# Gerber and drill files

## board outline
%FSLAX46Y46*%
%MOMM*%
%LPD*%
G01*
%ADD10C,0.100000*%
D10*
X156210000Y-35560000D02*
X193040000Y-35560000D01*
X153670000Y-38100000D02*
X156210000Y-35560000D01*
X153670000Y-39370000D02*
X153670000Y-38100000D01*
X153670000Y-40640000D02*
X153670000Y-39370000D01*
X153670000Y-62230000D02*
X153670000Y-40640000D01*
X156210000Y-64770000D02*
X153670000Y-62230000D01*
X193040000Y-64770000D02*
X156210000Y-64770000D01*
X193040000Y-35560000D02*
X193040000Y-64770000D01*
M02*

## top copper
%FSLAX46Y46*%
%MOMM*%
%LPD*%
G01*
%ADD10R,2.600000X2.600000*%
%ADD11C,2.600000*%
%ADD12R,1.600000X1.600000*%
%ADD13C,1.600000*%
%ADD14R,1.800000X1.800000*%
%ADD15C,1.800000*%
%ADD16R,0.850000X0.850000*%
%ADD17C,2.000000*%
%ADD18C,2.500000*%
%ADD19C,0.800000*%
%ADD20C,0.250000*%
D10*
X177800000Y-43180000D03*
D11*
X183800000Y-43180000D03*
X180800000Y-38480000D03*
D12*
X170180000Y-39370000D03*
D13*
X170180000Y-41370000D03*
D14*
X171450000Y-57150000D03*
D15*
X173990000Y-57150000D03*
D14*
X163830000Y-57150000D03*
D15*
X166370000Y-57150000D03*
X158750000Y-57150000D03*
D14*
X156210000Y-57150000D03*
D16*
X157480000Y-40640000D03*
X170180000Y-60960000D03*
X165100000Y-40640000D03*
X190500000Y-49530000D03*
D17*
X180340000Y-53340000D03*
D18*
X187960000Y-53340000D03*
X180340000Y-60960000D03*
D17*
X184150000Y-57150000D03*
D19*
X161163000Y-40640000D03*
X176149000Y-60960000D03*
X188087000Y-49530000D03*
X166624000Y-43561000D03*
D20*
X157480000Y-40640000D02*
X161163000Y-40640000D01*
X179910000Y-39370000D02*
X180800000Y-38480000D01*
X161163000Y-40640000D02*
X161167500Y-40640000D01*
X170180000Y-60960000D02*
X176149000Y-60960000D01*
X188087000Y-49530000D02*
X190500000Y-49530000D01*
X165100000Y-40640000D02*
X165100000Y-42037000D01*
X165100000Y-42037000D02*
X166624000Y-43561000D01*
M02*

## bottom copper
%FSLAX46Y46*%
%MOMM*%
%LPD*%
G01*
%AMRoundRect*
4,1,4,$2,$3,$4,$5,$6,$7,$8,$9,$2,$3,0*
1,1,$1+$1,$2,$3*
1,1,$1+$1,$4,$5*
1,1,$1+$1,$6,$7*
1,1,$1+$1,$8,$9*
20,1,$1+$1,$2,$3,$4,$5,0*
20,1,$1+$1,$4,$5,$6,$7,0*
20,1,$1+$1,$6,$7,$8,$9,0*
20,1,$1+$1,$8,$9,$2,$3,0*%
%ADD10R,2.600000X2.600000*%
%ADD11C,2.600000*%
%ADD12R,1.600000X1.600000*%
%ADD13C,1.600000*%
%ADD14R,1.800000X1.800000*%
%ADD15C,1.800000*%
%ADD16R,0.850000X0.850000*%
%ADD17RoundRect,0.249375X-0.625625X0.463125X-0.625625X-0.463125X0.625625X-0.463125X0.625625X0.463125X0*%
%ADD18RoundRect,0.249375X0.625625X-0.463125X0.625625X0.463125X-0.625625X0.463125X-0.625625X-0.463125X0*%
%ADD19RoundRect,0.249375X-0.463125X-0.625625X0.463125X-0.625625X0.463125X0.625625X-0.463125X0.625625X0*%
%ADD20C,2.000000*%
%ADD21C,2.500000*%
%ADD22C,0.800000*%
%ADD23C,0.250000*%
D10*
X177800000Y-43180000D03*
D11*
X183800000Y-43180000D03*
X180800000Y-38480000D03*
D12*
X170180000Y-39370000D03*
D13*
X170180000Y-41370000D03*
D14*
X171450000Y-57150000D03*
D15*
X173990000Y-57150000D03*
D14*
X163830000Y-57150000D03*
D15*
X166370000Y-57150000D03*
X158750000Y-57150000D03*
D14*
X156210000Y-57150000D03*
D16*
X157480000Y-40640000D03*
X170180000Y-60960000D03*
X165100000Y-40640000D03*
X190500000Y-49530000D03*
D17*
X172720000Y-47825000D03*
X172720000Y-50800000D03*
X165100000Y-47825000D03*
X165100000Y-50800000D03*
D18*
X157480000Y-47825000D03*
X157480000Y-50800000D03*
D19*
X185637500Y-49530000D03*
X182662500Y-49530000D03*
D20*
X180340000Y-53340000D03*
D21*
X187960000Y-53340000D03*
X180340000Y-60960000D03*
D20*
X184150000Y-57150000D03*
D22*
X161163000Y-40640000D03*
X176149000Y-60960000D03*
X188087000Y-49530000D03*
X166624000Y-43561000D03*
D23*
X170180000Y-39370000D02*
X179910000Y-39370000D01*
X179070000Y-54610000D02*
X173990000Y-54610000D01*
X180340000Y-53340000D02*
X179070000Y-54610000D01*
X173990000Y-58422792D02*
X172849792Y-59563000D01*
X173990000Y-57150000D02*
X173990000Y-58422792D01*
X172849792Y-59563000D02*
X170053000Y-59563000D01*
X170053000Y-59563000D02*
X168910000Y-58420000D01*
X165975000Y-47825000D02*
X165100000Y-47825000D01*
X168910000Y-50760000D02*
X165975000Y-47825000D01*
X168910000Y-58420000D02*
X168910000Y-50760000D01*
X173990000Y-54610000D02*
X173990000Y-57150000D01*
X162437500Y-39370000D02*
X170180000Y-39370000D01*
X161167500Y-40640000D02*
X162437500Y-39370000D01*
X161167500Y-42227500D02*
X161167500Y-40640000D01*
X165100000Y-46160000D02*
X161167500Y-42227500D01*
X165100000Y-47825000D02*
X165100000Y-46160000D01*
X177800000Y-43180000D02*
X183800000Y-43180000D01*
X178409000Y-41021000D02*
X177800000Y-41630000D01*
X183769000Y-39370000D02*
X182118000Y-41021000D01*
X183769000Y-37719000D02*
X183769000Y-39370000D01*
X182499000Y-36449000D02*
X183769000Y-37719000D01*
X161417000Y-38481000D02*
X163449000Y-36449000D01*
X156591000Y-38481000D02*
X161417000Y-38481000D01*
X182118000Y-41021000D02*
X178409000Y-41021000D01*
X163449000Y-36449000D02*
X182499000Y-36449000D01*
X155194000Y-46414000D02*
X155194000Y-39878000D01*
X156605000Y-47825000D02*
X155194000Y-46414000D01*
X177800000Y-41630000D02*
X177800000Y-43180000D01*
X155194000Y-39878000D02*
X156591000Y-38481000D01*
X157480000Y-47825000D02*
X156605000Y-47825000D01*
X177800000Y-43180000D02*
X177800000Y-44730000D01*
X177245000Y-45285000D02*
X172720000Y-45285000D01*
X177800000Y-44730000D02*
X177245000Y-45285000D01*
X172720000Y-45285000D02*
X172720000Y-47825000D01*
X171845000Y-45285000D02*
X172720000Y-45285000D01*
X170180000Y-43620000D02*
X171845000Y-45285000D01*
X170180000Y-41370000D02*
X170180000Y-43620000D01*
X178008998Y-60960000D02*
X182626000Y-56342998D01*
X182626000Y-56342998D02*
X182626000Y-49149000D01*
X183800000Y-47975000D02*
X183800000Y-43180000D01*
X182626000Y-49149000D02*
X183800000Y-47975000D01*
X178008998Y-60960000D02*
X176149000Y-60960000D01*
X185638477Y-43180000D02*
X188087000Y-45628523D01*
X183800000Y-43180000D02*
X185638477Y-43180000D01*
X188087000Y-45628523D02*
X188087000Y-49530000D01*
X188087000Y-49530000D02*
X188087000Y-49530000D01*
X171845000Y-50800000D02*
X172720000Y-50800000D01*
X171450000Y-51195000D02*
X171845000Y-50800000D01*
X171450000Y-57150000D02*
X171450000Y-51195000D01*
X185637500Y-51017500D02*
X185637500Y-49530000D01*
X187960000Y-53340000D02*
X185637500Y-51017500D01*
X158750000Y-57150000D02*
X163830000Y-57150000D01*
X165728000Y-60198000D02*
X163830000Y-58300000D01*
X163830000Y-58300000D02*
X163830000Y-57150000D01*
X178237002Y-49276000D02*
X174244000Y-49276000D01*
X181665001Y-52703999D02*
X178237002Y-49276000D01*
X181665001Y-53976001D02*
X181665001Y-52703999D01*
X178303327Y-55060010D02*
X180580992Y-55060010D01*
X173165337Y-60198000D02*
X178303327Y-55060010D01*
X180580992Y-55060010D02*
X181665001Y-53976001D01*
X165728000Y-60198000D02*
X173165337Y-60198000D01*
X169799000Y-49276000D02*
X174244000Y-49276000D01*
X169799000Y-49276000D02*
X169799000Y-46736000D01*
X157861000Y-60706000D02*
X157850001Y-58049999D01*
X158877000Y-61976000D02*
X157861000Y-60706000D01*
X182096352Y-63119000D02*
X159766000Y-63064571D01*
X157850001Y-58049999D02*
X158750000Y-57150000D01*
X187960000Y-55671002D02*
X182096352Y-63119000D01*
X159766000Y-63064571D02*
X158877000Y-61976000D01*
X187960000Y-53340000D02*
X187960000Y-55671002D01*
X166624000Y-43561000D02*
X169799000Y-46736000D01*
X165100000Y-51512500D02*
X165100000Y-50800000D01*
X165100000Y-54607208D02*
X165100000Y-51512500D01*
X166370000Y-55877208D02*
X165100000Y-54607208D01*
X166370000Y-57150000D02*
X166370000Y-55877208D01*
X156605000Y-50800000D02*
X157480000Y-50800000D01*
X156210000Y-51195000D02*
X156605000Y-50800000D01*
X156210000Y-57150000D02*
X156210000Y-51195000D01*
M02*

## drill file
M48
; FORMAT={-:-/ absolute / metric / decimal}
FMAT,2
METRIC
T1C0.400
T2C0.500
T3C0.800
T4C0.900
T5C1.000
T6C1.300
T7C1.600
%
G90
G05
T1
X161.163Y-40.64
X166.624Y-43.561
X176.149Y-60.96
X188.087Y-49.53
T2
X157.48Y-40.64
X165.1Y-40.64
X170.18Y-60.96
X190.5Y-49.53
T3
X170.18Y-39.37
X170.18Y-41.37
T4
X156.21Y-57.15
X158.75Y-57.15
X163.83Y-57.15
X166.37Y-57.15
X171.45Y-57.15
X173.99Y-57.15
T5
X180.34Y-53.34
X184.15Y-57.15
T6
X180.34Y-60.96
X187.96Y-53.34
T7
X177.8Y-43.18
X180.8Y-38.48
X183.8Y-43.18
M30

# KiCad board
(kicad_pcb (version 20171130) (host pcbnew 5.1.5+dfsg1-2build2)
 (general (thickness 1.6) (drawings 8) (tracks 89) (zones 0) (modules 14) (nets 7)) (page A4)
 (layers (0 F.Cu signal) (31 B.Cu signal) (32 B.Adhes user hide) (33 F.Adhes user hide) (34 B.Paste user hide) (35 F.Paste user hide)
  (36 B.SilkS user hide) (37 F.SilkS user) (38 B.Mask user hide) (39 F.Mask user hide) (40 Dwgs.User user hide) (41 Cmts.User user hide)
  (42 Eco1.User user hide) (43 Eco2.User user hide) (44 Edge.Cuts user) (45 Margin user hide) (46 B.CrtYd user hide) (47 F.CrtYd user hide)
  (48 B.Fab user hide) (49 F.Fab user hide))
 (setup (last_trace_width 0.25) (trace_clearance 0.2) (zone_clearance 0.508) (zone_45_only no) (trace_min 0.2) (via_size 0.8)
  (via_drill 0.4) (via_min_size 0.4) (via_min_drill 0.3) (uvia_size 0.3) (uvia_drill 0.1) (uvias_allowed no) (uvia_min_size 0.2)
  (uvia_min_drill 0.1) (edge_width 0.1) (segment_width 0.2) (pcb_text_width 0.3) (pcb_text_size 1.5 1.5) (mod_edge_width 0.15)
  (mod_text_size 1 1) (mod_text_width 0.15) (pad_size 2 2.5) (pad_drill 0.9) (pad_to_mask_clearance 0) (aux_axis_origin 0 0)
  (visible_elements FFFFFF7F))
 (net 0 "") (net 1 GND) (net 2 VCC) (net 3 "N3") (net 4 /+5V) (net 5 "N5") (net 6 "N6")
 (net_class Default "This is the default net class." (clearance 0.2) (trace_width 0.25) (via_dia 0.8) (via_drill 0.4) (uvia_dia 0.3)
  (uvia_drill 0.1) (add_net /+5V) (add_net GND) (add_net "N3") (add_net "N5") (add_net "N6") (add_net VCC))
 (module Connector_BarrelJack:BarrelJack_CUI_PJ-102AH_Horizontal (layer F.Cu) (at 177.8 43.18 90)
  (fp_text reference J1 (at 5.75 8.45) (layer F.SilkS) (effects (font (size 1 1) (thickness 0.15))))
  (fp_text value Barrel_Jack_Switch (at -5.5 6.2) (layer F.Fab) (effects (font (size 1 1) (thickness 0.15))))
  (pad 1 thru_hole rect (at 0 0 90) (size 2.6 2.6) (drill 1.6) (layers *.Cu *.Mask) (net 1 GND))
  (pad 2 thru_hole circle (at 0 6 90) (size 2.6 2.6) (drill 1.6) (layers *.Cu *.Mask) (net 1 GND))
  (pad 3 thru_hole circle (at 4.7 3 90) (size 2.6 2.6) (drill 1.6) (layers *.Cu *.Mask) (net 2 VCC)))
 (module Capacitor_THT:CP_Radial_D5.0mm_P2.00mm (layer F.Cu) (at 170.18 39.37 270)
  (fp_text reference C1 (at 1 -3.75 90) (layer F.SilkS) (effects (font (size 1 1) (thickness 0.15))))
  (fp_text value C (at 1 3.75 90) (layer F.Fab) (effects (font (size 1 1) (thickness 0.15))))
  (pad 1 thru_hole rect (at 0 0 270) (size 1.6 1.6) (drill 0.8) (layers *.Cu *.Mask) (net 2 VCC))
  (pad 2 thru_hole circle (at 2 0 270) (size 1.6 1.6) (drill 0.8) (layers *.Cu *.Mask) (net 1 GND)))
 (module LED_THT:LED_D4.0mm (layer F.Cu) (at 171.45 57.15)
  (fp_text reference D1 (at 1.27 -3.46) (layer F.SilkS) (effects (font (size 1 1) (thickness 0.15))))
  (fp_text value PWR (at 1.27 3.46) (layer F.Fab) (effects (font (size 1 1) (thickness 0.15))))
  (pad 1 thru_hole rect (at 0 0) (size 1.8 1.8) (drill 0.9) (layers *.Cu *.Mask) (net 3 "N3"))
  (pad 2 thru_hole circle (at 2.54 0) (size 1.8 1.8) (drill 0.9) (layers *.Cu *.Mask) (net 2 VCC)))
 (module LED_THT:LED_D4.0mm (layer F.Cu) (at 163.83 57.15)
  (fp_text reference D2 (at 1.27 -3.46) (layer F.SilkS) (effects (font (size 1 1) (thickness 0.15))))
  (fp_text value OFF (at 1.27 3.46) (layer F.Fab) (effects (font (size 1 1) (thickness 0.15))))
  (pad 1 thru_hole rect (at 0 0) (size 1.8 1.8) (drill 0.9) (layers *.Cu *.Mask) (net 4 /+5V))
  (pad 2 thru_hole circle (at 2.54 0) (size 1.8 1.8) (drill 0.9) (layers *.Cu *.Mask) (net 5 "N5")))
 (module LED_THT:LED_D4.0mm (layer F.Cu) (at 156.21 57.15)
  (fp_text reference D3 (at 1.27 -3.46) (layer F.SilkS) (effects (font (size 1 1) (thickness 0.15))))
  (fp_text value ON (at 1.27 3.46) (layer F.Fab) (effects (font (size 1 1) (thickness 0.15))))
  (pad 2 thru_hole circle (at 2.54 0) (size 1.8 1.8) (drill 0.9) (layers *.Cu *.Mask) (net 4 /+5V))
  (pad 1 thru_hole rect (at 0 0) (size 1.8 1.8) (drill 0.9) (layers *.Cu *.Mask) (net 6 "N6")))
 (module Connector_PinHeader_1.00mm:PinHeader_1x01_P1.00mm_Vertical (layer F.Cu) (at 157.48 40.64)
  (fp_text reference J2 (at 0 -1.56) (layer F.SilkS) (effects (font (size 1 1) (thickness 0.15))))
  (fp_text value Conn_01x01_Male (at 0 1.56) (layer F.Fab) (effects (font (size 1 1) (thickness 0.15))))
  (pad 1 thru_hole rect (at 0 0) (size 0.85 0.85) (drill 0.5) (layers *.Cu *.Mask) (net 2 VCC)))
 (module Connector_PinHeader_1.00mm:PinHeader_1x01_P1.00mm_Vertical (layer F.Cu) (at 170.18 60.96)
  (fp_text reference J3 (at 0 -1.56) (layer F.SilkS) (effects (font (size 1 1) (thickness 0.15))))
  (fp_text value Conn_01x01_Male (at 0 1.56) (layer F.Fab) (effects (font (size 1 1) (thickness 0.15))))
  (pad 1 thru_hole rect (at 0 0) (size 0.85 0.85) (drill 0.5) (layers *.Cu *.Mask) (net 1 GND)))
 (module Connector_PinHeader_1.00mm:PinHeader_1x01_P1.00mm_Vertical (layer F.Cu) (at 165.1 40.64)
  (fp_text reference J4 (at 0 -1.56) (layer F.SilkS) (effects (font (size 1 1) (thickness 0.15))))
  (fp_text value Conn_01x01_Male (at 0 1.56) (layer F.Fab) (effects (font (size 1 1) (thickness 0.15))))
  (pad 1 thru_hole rect (at 0 0) (size 0.85 0.85) (drill 0.5) (layers *.Cu *.Mask) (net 4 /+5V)))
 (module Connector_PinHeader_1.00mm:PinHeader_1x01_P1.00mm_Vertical (layer F.Cu) (at 190.5 49.53)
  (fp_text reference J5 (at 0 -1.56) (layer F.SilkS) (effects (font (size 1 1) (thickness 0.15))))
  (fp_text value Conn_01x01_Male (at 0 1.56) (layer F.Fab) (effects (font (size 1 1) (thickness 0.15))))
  (pad 1 thru_hole rect (at 0 0) (size 0.85 0.85) (drill 0.5) (layers *.Cu *.Mask) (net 1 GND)))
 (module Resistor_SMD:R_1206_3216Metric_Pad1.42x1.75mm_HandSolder (layer F.Cu) (at 172.72 49.3125 270)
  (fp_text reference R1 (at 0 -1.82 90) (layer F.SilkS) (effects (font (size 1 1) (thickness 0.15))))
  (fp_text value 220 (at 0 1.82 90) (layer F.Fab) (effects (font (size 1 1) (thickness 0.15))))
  (pad 1 smd roundrect (at -1.4875 0 270) (size 1.425 1.75) (layers B.Cu F.Paste F.Mask) (roundrect_rratio 0.175) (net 1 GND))
  (pad 2 smd roundrect (at 1.4875 0 270) (size 1.425 1.75) (layers B.Cu F.Paste F.Mask) (roundrect_rratio 0.175) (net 3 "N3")))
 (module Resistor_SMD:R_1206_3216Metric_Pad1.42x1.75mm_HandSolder (layer F.Cu) (at 165.1 49.3125 270)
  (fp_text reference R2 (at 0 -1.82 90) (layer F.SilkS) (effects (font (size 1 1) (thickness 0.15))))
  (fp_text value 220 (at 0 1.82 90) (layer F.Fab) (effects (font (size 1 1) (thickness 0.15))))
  (pad 1 smd roundrect (at -1.4875 0 270) (size 1.425 1.75) (layers B.Cu F.Paste F.Mask) (roundrect_rratio 0.175) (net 2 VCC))
  (pad 2 smd roundrect (at 1.4875 0 270) (size 1.425 1.75) (layers B.Cu F.Paste F.Mask) (roundrect_rratio 0.175) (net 5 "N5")))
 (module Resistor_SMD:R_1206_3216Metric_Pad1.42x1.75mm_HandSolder (layer F.Cu) (at 157.48 49.3125 90)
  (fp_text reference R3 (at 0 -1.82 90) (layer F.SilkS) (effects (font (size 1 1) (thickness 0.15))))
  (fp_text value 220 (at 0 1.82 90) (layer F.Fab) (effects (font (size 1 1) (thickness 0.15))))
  (pad 2 smd roundrect (at 1.4875 0 90) (size 1.425 1.75) (layers B.Cu F.Paste F.Mask) (roundrect_rratio 0.175) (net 1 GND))
  (pad 1 smd roundrect (at -1.4875 0 90) (size 1.425 1.75) (layers B.Cu F.Paste F.Mask) (roundrect_rratio 0.175) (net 6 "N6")))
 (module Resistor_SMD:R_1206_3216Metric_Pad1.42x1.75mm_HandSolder (layer F.Cu) (at 184.15 49.53)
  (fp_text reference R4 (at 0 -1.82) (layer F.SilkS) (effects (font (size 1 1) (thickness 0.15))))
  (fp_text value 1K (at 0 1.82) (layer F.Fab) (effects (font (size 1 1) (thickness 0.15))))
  (pad 2 smd roundrect (at 1.4875 0) (size 1.425 1.75) (layers B.Cu F.Paste F.Mask) (roundrect_rratio 0.175) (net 4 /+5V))
  (pad 1 smd roundrect (at -1.4875 0) (size 1.425 1.75) (layers B.Cu F.Paste F.Mask) (roundrect_rratio 0.175) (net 1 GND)))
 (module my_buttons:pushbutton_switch (layer F.Cu) (at 184.15 49.53)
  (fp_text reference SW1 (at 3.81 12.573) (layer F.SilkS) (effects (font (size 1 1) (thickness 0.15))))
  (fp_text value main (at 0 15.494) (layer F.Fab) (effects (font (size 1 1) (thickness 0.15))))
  (pad 1 thru_hole circle (at -3.81 3.81) (size 2 2) (drill 1) (layers *.Cu *.Mask) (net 2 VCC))
  (pad 2 thru_hole circle (at 3.81 3.81) (size 2.5 2.5) (drill 1.3) (layers *.Cu *.Mask) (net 4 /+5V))
  (pad 3 thru_hole circle (at -3.81 11.43) (size 2.5 2.5) (drill 1.3) (layers *.Cu *.Mask))
  (pad 4 thru_hole circle (at 0 7.62) (size 2 2) (drill 1) (layers *.Cu *.Mask)))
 (gr_line (start 156.21 35.56) (end 193.04 35.56) (layer Edge.Cuts) (width 0.1))
 (gr_line (start 153.67 38.1) (end 156.21 35.56) (layer Edge.Cuts) (width 0.1))
 (gr_line (start 153.67 39.37) (end 153.67 38.1) (layer Edge.Cuts) (width 0.1))
 (gr_line (start 153.67 40.64) (end 153.67 39.37) (layer Edge.Cuts) (width 0.1))
 (gr_line (start 153.67 62.23) (end 153.67 40.64) (layer Edge.Cuts) (width 0.1))
 (gr_line (start 156.21 64.77) (end 153.67 62.23) (layer Edge.Cuts) (width 0.1))
 (gr_line (start 193.04 64.77) (end 156.21 64.77) (layer Edge.Cuts) (width 0.1))
 (gr_line (start 193.04 35.56) (end 193.04 64.77) (layer Edge.Cuts) (width 0.1))
 (segment (start 157.48 40.64) (end 161.163 40.64) (width 0.25) (layer F.Cu) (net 2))
 (segment (start 179.91 39.37) (end 180.8 38.48) (width 0.25) (layer F.Cu) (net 2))
 (segment (start 170.18 39.37) (end 179.91 39.37) (width 0.25) (layer B.Cu) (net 2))
 (segment (start 179.07 54.61) (end 173.99 54.61) (width 0.25) (layer B.Cu) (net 2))
 (segment (start 180.34 53.34) (end 179.07 54.61) (width 0.25) (layer B.Cu) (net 2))
 (segment (start 173.99 58.422792) (end 172.849792 59.563) (width 0.25) (layer B.Cu) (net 2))
 (segment (start 173.99 57.15) (end 173.99 58.422792) (width 0.25) (layer B.Cu) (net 2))
 (segment (start 172.849792 59.563) (end 170.053 59.563) (width 0.25) (layer B.Cu) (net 2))
 (segment (start 170.053 59.563) (end 168.91 58.42) (width 0.25) (layer B.Cu) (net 2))
 (segment (start 165.975 47.825) (end 165.1 47.825) (width 0.25) (layer B.Cu) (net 2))
 (segment (start 168.91 50.76) (end 165.975 47.825) (width 0.25) (layer B.Cu) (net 2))
 (segment (start 168.91 58.42) (end 168.91 50.76) (width 0.25) (layer B.Cu) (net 2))
 (segment (start 173.99 54.61) (end 173.99 57.15) (width 0.25) (layer B.Cu) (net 2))
 (segment (start 162.4375 39.37) (end 170.18 39.37) (width 0.25) (layer B.Cu) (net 2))
 (segment (start 161.1675 40.64) (end 162.4375 39.37) (width 0.25) (layer B.Cu) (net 2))
 (segment (start 161.1675 42.2275) (end 161.1675 40.64) (width 0.25) (layer B.Cu) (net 2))
 (segment (start 165.1 46.16) (end 161.1675 42.2275) (width 0.25) (layer B.Cu) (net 2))
 (segment (start 165.1 47.825) (end 165.1 46.16) (width 0.25) (layer B.Cu) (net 2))
 (segment (start 161.163 40.64) (end 161.1675 40.64) (width 0.25) (layer F.Cu) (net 2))
 (via (at 161.163 40.64) (size 0.8) (drill 0.4) (layers F.Cu B.Cu) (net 2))
 (segment (start 177.8 43.18) (end 183.8 43.18) (width 0.25) (layer B.Cu) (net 1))
 (segment (start 178.409 41.021) (end 177.8 41.63) (width 0.25) (layer B.Cu) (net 1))
 (segment (start 183.769 39.37) (end 182.118 41.021) (width 0.25) (layer B.Cu) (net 1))
 (segment (start 183.769 37.719) (end 183.769 39.37) (width 0.25) (layer B.Cu) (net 1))
 (segment (start 182.499 36.449) (end 183.769 37.719) (width 0.25) (layer B.Cu) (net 1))
 (segment (start 161.417 38.481) (end 163.449 36.449) (width 0.25) (layer B.Cu) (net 1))
 (segment (start 156.591 38.481) (end 161.417 38.481) (width 0.25) (layer B.Cu) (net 1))
 (segment (start 182.118 41.021) (end 178.409 41.021) (width 0.25) (layer B.Cu) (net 1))
 (segment (start 163.449 36.449) (end 182.499 36.449) (width 0.25) (layer B.Cu) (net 1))
 (segment (start 155.194 46.414) (end 155.194 39.878) (width 0.25) (layer B.Cu) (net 1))
 (segment (start 156.605 47.825) (end 155.194 46.414) (width 0.25) (layer B.Cu) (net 1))
 (segment (start 177.8 41.63) (end 177.8 43.18) (width 0.25) (layer B.Cu) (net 1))
 (segment (start 155.194 39.878) (end 156.591 38.481) (width 0.25) (layer B.Cu) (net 1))
 (segment (start 157.48 47.825) (end 156.605 47.825) (width 0.25) (layer B.Cu) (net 1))
 (segment (start 177.8 43.18) (end 177.8 44.73) (width 0.25) (layer B.Cu) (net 1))
 (segment (start 177.245 45.285) (end 172.72 45.285) (width 0.25) (layer B.Cu) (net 1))
 (segment (start 177.8 44.73) (end 177.245 45.285) (width 0.25) (layer B.Cu) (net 1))
 (segment (start 172.72 45.285) (end 172.72 47.825) (width 0.25) (layer B.Cu) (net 1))
 (segment (start 171.845 45.285) (end 172.72 45.285) (width 0.25) (layer B.Cu) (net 1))
 (segment (start 170.18 43.62) (end 171.845 45.285) (width 0.25) (layer B.Cu) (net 1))
 (segment (start 170.18 41.37) (end 170.18 43.62) (width 0.25) (layer B.Cu) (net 1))
 (segment (start 178.008998 60.96) (end 182.626 56.342998) (width 0.25) (layer B.Cu) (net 1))
 (segment (start 170.18 60.96) (end 176.149 60.96) (width 0.25) (layer F.Cu) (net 1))
 (segment (start 182.626 56.342998) (end 182.626 49.149) (width 0.25) (layer B.Cu) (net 1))
 (segment (start 183.8 47.975) (end 183.8 43.18) (width 0.25) (layer B.Cu) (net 1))
 (segment (start 182.626 49.149) (end 183.8 47.975) (width 0.25) (layer B.Cu) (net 1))
 (via (at 176.149 60.96) (size 0.8) (drill 0.4) (layers F.Cu B.Cu) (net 1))
 (segment (start 178.008998 60.96) (end 176.149 60.96) (width 0.25) (layer B.Cu) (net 1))
 (segment (start 185.638477 43.18) (end 188.087 45.628523) (width 0.25) (layer B.Cu) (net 1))
 (segment (start 183.8 43.18) (end 185.638477 43.18) (width 0.25) (layer B.Cu) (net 1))
 (segment (start 188.087 45.628523) (end 188.087 49.53) (width 0.25) (layer B.Cu) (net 1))
 (segment (start 188.087 49.53) (end 190.5 49.53) (width 0.25) (layer F.Cu) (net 1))
 (segment (start 188.087 49.53) (end 188.087 49.53) (width 0.25) (layer B.Cu) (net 1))
 (via (at 188.087 49.53) (size 0.8) (drill 0.4) (layers F.Cu B.Cu) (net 1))
 (segment (start 171.845 50.8) (end 172.72 50.8) (width 0.25) (layer B.Cu) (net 3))
 (segment (start 171.45 51.195) (end 171.845 50.8) (width 0.25) (layer B.Cu) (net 3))
 (segment (start 171.45 57.15) (end 171.45 51.195) (width 0.25) (layer B.Cu) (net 3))
 (segment (start 185.6375 51.0175) (end 185.6375 49.53) (width 0.25) (layer B.Cu) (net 4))
 (segment (start 187.96 53.34) (end 185.6375 51.0175) (width 0.25) (layer B.Cu) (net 4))
 (segment (start 158.75 57.15) (end 163.83 57.15) (width 0.25) (layer B.Cu) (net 4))
 (segment (start 165.1 40.64) (end 165.1 42.037) (width 0.25) (layer F.Cu) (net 4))
 (segment (start 165.1 42.037) (end 166.624 43.561) (width 0.25) (layer F.Cu) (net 4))
 (segment (start 165.728 60.198) (end 163.83 58.3) (width 0.25) (layer B.Cu) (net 4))
 (segment (start 163.83 58.3) (end 163.83 57.15) (width 0.25) (layer B.Cu) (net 4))
 (segment (start 178.237002 49.276) (end 174.244 49.276) (width 0.25) (layer B.Cu) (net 4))
 (segment (start 181.665001 52.703999) (end 178.237002 49.276) (width 0.25) (layer B.Cu) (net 4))
 (segment (start 181.665001 53.976001) (end 181.665001 52.703999) (width 0.25) (layer B.Cu) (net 4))
 (segment (start 178.303327 55.06001) (end 180.580992 55.06001) (width 0.25) (layer B.Cu) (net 4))
 (segment (start 173.165337 60.198) (end 178.303327 55.06001) (width 0.25) (layer B.Cu) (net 4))
 (segment (start 180.580992 55.06001) (end 181.665001 53.976001) (width 0.25) (layer B.Cu) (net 4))
 (segment (start 165.728 60.198) (end 173.165337 60.198) (width 0.25) (layer B.Cu) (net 4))
 (segment (start 169.799 49.276) (end 174.244 49.276) (width 0.25) (layer B.Cu) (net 4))
 (segment (start 169.799 49.276) (end 169.799 46.736) (width 0.25) (layer B.Cu) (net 4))
 (segment (start 157.861 60.706) (end 157.850001 58.049999) (width 0.25) (layer B.Cu) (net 4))
 (segment (start 158.877 61.976) (end 157.861 60.706) (width 0.25) (layer B.Cu) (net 4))
 (segment (start 182.096352 63.119) (end 159.766 63.064571) (width 0.25) (layer B.Cu) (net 4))
 (segment (start 157.850001 58.049999) (end 158.75 57.15) (width 0.25) (layer B.Cu) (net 4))
 (segment (start 187.96 55.671002) (end 182.096352 63.119) (width 0.25) (layer B.Cu) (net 4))
 (segment (start 159.766 63.064571) (end 158.877 61.976) (width 0.25) (layer B.Cu) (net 4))
 (segment (start 187.96 53.34) (end 187.96 55.671002) (width 0.25) (layer B.Cu) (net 4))
 (segment (start 166.624 43.561) (end 169.799 46.736) (width 0.25) (layer B.Cu) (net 4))
 (via (at 166.624 43.561) (size 0.8) (drill 0.4) (layers F.Cu B.Cu) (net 4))
 (segment (start 165.1 51.5125) (end 165.1 50.8) (width 0.25) (layer B.Cu) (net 5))
 (segment (start 165.1 54.607208) (end 165.1 51.5125) (width 0.25) (layer B.Cu) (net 5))
 (segment (start 166.37 55.877208) (end 165.1 54.607208) (width 0.25) (layer B.Cu) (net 5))
 (segment (start 166.37 57.15) (end 166.37 55.877208) (width 0.25) (layer B.Cu) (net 5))
 (segment (start 156.605 50.8) (end 157.48 50.8) (width 0.25) (layer B.Cu) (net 6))
 (segment (start 156.21 51.195) (end 156.605 50.8) (width 0.25) (layer B.Cu) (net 6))
 (segment (start 156.21 57.15) (end 156.21 51.195) (width 0.25) (layer B.Cu) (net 6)))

